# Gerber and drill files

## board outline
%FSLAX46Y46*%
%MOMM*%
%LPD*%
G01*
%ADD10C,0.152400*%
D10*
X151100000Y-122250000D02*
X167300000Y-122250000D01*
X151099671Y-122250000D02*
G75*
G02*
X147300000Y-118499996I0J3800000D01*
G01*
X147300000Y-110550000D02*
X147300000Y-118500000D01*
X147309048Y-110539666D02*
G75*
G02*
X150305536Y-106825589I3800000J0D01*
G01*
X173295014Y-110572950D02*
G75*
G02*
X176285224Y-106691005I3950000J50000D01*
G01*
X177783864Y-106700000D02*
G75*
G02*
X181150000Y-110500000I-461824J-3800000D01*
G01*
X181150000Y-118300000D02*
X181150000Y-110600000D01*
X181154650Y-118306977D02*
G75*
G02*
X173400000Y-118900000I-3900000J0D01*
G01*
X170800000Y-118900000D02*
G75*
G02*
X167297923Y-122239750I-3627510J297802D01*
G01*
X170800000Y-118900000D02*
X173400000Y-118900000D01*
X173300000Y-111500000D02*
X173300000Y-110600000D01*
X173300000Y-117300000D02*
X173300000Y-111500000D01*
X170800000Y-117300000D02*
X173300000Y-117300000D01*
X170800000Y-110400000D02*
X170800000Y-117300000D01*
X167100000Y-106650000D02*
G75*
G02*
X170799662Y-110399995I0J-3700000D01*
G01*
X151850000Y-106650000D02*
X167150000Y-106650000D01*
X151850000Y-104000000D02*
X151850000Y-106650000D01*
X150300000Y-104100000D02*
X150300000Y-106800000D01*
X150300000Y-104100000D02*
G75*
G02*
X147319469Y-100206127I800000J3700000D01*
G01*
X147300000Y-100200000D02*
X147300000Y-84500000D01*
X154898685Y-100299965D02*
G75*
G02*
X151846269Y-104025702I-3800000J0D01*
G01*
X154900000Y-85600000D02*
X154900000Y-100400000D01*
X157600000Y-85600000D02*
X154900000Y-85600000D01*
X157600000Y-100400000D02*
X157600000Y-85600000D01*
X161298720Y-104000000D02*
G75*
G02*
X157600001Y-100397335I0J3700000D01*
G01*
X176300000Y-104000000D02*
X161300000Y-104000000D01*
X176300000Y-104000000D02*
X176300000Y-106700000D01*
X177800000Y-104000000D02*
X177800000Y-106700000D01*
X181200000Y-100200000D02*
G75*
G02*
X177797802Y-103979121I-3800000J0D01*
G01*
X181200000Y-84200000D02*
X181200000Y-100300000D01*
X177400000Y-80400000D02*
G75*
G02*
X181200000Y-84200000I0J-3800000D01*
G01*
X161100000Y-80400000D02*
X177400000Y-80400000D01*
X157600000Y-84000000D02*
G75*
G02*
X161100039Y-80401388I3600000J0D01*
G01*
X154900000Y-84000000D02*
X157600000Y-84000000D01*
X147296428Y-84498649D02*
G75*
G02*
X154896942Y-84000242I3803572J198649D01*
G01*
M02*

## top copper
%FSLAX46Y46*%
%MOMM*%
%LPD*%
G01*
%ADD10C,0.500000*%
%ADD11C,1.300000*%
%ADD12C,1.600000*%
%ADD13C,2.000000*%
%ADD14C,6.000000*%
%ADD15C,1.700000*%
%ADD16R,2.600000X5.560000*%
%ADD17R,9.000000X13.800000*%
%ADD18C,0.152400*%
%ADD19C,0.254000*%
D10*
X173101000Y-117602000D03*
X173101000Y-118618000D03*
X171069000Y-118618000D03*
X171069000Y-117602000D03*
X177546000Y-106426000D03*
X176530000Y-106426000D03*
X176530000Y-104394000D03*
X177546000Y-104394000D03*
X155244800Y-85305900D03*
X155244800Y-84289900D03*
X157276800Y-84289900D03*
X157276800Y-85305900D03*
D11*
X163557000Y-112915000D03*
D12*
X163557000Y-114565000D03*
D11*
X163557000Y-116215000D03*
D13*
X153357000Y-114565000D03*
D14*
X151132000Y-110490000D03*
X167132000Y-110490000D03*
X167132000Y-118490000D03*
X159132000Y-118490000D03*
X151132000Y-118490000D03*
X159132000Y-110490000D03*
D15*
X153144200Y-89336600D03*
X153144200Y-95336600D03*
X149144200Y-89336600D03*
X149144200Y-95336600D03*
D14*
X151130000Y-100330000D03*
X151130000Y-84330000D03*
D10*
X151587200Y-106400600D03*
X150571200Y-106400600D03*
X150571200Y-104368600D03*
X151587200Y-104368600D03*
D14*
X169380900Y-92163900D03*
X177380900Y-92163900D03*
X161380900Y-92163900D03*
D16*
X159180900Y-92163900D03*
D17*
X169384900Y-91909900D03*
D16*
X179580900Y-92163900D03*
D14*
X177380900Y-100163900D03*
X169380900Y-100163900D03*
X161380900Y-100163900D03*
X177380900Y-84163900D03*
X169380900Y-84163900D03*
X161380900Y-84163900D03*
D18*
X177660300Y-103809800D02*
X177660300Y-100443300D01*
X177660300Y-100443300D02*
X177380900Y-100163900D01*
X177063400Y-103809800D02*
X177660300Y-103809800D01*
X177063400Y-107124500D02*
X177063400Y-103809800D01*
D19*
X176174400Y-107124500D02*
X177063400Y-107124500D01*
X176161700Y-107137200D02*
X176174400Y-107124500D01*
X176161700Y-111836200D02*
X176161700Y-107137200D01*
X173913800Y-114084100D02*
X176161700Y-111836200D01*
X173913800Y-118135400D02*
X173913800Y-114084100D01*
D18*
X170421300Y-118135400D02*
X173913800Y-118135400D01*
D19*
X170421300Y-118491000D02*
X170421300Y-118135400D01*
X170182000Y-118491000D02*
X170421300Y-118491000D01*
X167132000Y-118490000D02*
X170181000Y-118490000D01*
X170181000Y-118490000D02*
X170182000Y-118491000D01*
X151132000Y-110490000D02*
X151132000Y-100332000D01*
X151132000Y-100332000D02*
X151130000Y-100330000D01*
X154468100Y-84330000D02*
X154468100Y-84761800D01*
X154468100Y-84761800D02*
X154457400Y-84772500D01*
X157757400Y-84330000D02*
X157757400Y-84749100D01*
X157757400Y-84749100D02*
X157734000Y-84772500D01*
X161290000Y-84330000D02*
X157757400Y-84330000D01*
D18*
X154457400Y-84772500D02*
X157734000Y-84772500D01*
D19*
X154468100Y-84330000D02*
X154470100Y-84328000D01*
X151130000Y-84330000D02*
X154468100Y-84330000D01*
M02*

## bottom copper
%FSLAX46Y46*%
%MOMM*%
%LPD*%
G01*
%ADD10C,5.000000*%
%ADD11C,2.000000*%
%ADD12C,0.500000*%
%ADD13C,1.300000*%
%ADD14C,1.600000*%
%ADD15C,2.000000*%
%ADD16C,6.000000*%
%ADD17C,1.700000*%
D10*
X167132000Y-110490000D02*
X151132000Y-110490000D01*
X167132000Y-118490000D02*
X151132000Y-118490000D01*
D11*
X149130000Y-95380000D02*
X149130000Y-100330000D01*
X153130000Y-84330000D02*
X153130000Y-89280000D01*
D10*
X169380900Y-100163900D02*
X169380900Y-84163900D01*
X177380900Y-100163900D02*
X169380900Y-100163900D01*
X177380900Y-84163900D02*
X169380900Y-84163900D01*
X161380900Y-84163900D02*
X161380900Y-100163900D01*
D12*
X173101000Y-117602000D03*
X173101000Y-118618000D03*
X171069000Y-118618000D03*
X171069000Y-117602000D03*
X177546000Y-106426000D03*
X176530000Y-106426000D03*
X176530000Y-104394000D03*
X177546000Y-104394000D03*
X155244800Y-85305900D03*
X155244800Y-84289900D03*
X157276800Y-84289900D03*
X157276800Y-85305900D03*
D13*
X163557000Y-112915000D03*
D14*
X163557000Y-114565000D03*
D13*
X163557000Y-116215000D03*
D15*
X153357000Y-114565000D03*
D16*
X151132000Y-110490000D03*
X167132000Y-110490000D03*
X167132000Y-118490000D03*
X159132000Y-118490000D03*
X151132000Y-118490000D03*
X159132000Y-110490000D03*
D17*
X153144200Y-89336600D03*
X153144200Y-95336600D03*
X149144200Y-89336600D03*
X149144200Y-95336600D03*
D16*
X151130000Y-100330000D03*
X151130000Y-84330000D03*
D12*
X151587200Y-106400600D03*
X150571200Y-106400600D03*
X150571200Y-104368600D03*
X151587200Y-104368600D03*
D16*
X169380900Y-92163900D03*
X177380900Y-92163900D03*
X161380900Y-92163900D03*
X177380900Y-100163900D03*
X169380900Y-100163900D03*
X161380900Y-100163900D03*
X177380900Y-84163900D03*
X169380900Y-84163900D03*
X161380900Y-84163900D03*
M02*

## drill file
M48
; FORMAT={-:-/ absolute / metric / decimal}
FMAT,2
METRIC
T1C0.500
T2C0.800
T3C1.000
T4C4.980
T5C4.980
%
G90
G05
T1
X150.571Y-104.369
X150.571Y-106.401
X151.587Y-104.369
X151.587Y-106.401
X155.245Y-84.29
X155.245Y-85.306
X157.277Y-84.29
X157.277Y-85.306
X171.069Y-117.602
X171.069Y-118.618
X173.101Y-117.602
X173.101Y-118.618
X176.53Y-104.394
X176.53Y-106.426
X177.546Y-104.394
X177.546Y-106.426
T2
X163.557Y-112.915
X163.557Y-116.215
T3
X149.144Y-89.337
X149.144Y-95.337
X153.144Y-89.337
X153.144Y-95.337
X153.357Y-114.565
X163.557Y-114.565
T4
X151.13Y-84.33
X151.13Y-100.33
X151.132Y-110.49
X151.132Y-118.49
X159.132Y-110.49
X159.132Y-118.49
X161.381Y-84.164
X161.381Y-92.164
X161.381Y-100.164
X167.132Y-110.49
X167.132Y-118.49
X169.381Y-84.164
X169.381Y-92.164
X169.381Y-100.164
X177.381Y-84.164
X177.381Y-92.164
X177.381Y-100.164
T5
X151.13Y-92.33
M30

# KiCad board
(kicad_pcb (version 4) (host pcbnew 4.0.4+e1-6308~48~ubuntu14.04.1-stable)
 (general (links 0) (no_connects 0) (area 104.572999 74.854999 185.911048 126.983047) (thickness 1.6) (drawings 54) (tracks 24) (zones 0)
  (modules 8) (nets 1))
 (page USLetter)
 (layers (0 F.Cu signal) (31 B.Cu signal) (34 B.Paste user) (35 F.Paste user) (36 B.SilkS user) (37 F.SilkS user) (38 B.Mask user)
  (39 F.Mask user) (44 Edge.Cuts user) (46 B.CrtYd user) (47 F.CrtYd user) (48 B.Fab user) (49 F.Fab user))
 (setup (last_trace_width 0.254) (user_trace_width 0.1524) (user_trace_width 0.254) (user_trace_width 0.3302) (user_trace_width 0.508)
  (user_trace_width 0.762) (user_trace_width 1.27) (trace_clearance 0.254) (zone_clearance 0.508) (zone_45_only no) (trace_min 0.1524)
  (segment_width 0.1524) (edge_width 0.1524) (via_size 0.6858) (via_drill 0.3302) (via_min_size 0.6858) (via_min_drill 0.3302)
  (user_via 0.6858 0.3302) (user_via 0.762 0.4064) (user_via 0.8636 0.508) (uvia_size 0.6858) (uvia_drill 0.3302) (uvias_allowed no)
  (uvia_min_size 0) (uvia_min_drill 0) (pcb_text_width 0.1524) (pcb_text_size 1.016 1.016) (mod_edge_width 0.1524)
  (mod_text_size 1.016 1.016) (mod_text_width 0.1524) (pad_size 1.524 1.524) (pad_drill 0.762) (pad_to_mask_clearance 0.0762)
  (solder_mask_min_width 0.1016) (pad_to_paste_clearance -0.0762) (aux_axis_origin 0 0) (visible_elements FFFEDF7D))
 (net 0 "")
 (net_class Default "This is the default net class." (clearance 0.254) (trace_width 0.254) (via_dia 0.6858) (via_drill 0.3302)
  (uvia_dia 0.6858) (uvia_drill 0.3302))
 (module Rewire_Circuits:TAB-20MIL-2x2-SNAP (layer F.Cu) (at 172.085 118.11 270)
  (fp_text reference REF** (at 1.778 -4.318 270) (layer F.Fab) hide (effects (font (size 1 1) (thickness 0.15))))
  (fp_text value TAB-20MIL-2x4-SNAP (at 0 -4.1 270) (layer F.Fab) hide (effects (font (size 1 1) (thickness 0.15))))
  (pad 1 thru_hole circle (at -0.508 -1.016 270) (size 0.5 0.5) (drill 0.5) (layers *.Cu))
  (pad 1 thru_hole circle (at 0.508 -1.016 270) (size 0.5 0.5) (drill 0.5) (layers *.Cu))
  (pad 1 thru_hole circle (at 0.508 1.016 270) (size 0.5 0.5) (drill 0.5) (layers *.Cu))
  (pad 1 thru_hole circle (at -0.508 1.016 270) (size 0.5 0.5) (drill 0.5) (layers *.Cu)))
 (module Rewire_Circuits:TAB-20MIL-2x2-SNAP (layer F.Cu) (at 177.038 105.41 180)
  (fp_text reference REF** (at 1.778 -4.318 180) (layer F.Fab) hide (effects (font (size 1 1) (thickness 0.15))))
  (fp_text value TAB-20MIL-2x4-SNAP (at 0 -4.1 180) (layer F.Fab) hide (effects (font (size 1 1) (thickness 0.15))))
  (pad 1 thru_hole circle (at -0.508 -1.016 180) (size 0.5 0.5) (drill 0.5) (layers *.Cu))
  (pad 1 thru_hole circle (at 0.508 -1.016 180) (size 0.5 0.5) (drill 0.5) (layers *.Cu))
  (pad 1 thru_hole circle (at 0.508 1.016 180) (size 0.5 0.5) (drill 0.5) (layers *.Cu))
  (pad 1 thru_hole circle (at -0.508 1.016 180) (size 0.5 0.5) (drill 0.5) (layers *.Cu)))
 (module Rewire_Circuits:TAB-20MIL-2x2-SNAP (layer F.Cu) (at 156.2608 84.7979 90)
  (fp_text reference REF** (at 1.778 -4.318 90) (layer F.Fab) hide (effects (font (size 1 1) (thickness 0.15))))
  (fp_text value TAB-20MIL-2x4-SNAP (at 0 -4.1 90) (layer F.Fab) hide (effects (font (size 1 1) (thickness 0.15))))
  (pad 1 thru_hole circle (at -0.508 -1.016 90) (size 0.5 0.5) (drill 0.5) (layers *.Cu))
  (pad 1 thru_hole circle (at 0.508 -1.016 90) (size 0.5 0.5) (drill 0.5) (layers *.Cu))
  (pad 1 thru_hole circle (at 0.508 1.016 90) (size 0.5 0.5) (drill 0.5) (layers *.Cu))
  (pad 1 thru_hole circle (at -0.508 1.016 90) (size 0.5 0.5) (drill 0.5) (layers *.Cu)))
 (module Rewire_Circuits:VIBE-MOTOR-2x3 (layer F.Cu) (at 167.132 110.49 180)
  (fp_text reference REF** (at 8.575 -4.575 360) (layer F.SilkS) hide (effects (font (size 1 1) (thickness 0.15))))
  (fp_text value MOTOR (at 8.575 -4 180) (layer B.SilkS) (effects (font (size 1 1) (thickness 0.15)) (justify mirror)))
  (fp_line (start 0 0) (end 16 0) (layer B.Cu) (width 5)) (fp_line (start 0 -8) (end 16 -8) (layer B.Cu) (width 5))
  (pad 1 thru_hole circle (at 3.575 -2.425 270) (size 1.3 1.3) (drill 0.8) (layers *.Cu *.Mask F.SilkS))
  (pad 3 thru_hole circle (at 3.575 -4.075 270) (size 1.6 1.6) (drill 1) (layers *.Cu *.Mask F.SilkS))
  (pad 2 thru_hole circle (at 3.575 -5.725 270) (size 1.3 1.3) (drill 0.8) (layers *.Cu *.Mask F.SilkS))
  (pad 3 thru_hole circle (at 13.775 -4.075 270) (size 2 2) (drill 1) (layers *.Cu *.Mask F.SilkS))
  (pad 1 thru_hole circle (at 16 0 180) (size 6 6) (drill 4.98) (layers *.Cu *.Mask))
  (pad 1 thru_hole circle (at 0 0 180) (size 6 6) (drill 4.98) (layers *.Cu *.Mask))
  (pad 2 thru_hole circle (at 0 -8 180) (size 6 6) (drill 4.98) (layers *.Cu *.Mask))
  (pad 2 thru_hole circle (at 8 -8 180) (size 6 6) (drill 4.98) (layers *.Cu *.Mask))
  (pad 2 thru_hole circle (at 16 -8 180) (size 6 6) (drill 4.98) (layers *.Cu *.Mask))
  (pad 1 thru_hole circle (at 8 0 180) (size 6 6) (drill 4.98) (layers *.Cu *.Mask)))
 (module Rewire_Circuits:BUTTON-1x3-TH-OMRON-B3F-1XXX (layer F.Cu) (at 151.13 100.33 90)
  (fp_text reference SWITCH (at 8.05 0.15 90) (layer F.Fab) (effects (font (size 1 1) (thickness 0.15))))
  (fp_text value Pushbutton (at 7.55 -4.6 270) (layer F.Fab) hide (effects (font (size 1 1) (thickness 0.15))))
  (fp_line (start 4.95 -2) (end 0 -2) (layer B.Cu) (width 2)) (fp_line (start 16 2) (end 11.05 2) (layer B.Cu) (width 2))
  (pad 2 thru_hole circle (at 10.9934 2.0142 90) (size 1.7 1.7) (drill 1) (layers *.Cu *.Mask))
  (pad 2 thru_hole circle (at 4.9934 2.0142 90) (size 1.7 1.7) (drill 1) (layers *.Cu *.Mask))
  (pad 1 thru_hole circle (at 10.9934 -1.9858 90) (size 1.7 1.7) (drill 1) (layers *.Cu *.Mask))
  (pad 1 thru_hole circle (at 4.9934 -1.9858 90) (size 1.7 1.7) (drill 1) (layers *.Cu *.Mask))
  (pad "" np_thru_hole circle (at 8 0 90) (size 4.88 4.88) (drill 4.98) (layers *.Cu *.Mask F.SilkS))
  (pad 1 thru_hole circle (at 0 0 90) (size 6 6) (drill 4.98) (layers *.Cu *.Mask F.SilkS))
  (pad 2 thru_hole circle (at 16 0 90) (size 6 6) (drill 4.98) (layers *.Cu *.Mask F.SilkS)))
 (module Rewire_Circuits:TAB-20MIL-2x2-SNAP (layer F.Cu) (at 151.0792 105.3846 180)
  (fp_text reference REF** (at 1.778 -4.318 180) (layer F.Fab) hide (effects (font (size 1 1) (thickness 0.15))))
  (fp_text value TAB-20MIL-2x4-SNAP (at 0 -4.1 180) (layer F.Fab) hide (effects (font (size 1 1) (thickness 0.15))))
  (pad 1 thru_hole circle (at -0.508 -1.016 180) (size 0.5 0.5) (drill 0.5) (layers *.Cu))
  (pad 1 thru_hole circle (at 0.508 -1.016 180) (size 0.5 0.5) (drill 0.5) (layers *.Cu))
  (pad 1 thru_hole circle (at 0.508 1.016 180) (size 0.5 0.5) (drill 0.5) (layers *.Cu))
  (pad 1 thru_hole circle (at -0.508 1.016 180) (size 0.5 0.5) (drill 0.5) (layers *.Cu)))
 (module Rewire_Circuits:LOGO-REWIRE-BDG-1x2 (layer F.Cu) (at 181.1528 114.427 90)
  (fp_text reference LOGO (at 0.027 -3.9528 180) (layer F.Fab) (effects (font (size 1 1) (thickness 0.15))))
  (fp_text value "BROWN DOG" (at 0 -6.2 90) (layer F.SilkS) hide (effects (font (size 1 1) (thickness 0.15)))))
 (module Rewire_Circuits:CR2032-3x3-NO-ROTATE (layer F.Cu) (at 177.3809 84.1639 180)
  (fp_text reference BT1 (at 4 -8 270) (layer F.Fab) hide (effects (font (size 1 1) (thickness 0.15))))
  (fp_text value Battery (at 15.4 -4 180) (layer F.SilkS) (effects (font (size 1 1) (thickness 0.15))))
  (fp_line (start 8 -16) (end 8 0) (layer B.Cu) (width 5)) (fp_line (start 0 -16) (end 8 -16) (layer B.Cu) (width 5))
  (fp_line (start 0 0) (end 8 0) (layer B.Cu) (width 5)) (fp_line (start 16 0) (end 16 -16) (layer B.Cu) (width 5))
  (pad GND thru_hole circle (at 8 -8 180) (size 6 6) (drill 4.98) (layers *.Cu *.Mask))
  (pad + thru_hole circle (at 0 -8 180) (size 6 6) (drill 4.98) (layers *.Cu *.Mask))
  (pad + thru_hole circle (at 16 -8 180) (size 6 6) (drill 4.98) (layers *.Cu *.Mask))
  (pad + smd rect (at 18.2 -8 180) (size 2.6 5.56) (layers F.Cu F.Paste F.Mask))
  (pad GND smd rect (at 7.996 -7.746 180) (size 9 13.8) (layers F.Cu F.Paste F.Mask))
  (pad + smd rect (at -2.2 -8 180) (size 2.6 5.56) (layers F.Cu F.Paste F.Mask))
  (pad GND thru_hole circle (at 0 -16 180) (size 6 6) (drill 4.98) (layers *.Cu *.Mask))
  (pad GND thru_hole circle (at 8 -16 180) (size 6 6) (drill 4.98) (layers *.Cu *.Mask))
  (pad + thru_hole circle (at 16 -16 180) (size 6 6) (drill 4.98) (layers *.Cu B.Mask))
  (pad GND thru_hole circle (at 0 0 180) (size 6 6) (drill 4.98) (layers *.Cu *.Mask))
  (pad GND thru_hole circle (at 8 0 180) (size 6 6) (drill 4.98) (layers *.Cu *.Mask))
  (pad + thru_hole circle (at 16 0 180) (size 6 6) (drill 4.98) (layers *.Cu B.Mask)))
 (gr_line (start 151.1 122.25) (end 167.3 122.25) (layer Edge.Cuts) (width 0.1524))
 (gr_arc (start 151.099671 118.45) (end 151.099671 122.25) (angle 89.24615167) (layer Edge.Cuts) (width 0.1524))
 (gr_line (start 147.3 110.55) (end 147.3 118.5) (layer Edge.Cuts) (width 0.1524))
 (gr_arc (start 151.109048 110.539666) (end 147.309048 110.539666) (angle 77.79262944) (layer Edge.Cuts) (width 0.1524))
 (gr_arc (start 177.245014 110.52295) (end 173.295014 110.57295) (angle 76.66359666) (layer Edge.Cuts) (width 0.1524))
 (gr_arc (start 177.32204 110.5) (end 177.783864 106.7) (angle 83.07067559) (layer Edge.Cuts) (width 0.1524))
 (gr_line (start 181.15 118.3) (end 181.15 110.6) (layer Edge.Cuts) (width 0.1524))
 (gr_arc (start 177.25465 118.306977) (end 181.15465 118.306977) (angle 171.2538377) (layer Edge.Cuts) (width 0.1524))
 (gr_arc (start 167.17249 118.602198) (end 170.8 118.9) (angle 83.33186569) (layer Edge.Cuts) (width 0.1524))
 (gr_line (start 170.8 118.9) (end 173.4 118.9) (layer Edge.Cuts) (width 0.1524))
 (gr_line (start 173.3 111.5) (end 173.3 110.6) (layer Edge.Cuts) (width 0.1524))
 (gr_line (start 173.3 117.3) (end 173.3 111.5) (layer Edge.Cuts) (width 0.1524))
 (gr_line (start 170.8 117.3) (end 173.3 117.3) (layer Edge.Cuts) (width 0.1524))
 (gr_line (start 170.8 110.4) (end 170.8 117.3) (layer Edge.Cuts) (width 0.1524))
 (gr_arc (start 167.1 110.35) (end 167.1 106.65) (angle 90.77421347) (layer Edge.Cuts) (width 0.1524))
 (gr_line (start 151.85 106.65) (end 167.15 106.65) (layer Edge.Cuts) (width 0.1524))
 (gr_line (start 151.85 104) (end 151.85 106.65) (layer Edge.Cuts) (width 0.1524))
 (gr_line (start 150.3 104.1) (end 150.3 106.8) (layer Edge.Cuts) (width 0.1524))
 (gr_arc (start 151.1 100.4) (end 150.3 104.1) (angle 80.73520472) (layer Edge.Cuts) (width 0.1524))
 (gr_line (start 147.3 100.2) (end 147.3 84.5) (layer Edge.Cuts) (width 0.1524))
 (gr_arc (start 151.098685 100.299965) (end 154.898685 100.299965) (angle 78.6540423) (layer Edge.Cuts) (width 0.1524))
 (gr_line (start 154.9 85.6) (end 154.9 100.4) (layer Edge.Cuts) (width 0.1524))
 (gr_line (start 157.6 85.6) (end 154.9 85.6) (layer Edge.Cuts) (width 0.1524))
 (gr_line (start 157.6 100.4) (end 157.6 85.6) (layer Edge.Cuts) (width 0.1524))
 (gr_arc (start 161.29872 100.3) (end 161.29872 104) (angle 88.49256424) (layer Edge.Cuts) (width 0.1524))
 (gr_line (start 176.3 104) (end 161.3 104) (layer Edge.Cuts) (width 0.1524))
 (gr_line (start 176.3 104) (end 176.3 106.7) (layer Edge.Cuts) (width 0.1524))
 (gr_line (start 177.8 104) (end 177.8 106.7) (layer Edge.Cuts) (width 0.1524))
 (gr_arc (start 177.4 100.2) (end 181.2 100.2) (angle 83.99099562) (layer Edge.Cuts) (width 0.1524))
 (gr_line (start 181.2 84.2) (end 181.2 100.3) (layer Edge.Cuts) (width 0.1524))
 (gr_arc (start 177.4 84.2) (end 177.4 80.4) (angle 90) (layer Edge.Cuts) (width 0.1524))
 (gr_line (start 161.1 80.4) (end 177.4 80.4) (layer Edge.Cuts) (width 0.1524))
 (gr_arc (start 161.2 84) (end 157.6 84) (angle 88.40885973) (layer Edge.Cuts) (width 0.1524))
 (gr_line (start 154.9 84) (end 157.6 84) (layer Edge.Cuts) (width 0.1524))
 (gr_arc (start 151.1 84.3) (end 147.296428 84.498649) (angle 178.4756859) (layer Edge.Cuts) (width 0.1524))
 (segment (start 177.6603 103.8098) (end 177.6603 100.4433) (width 0.1524) (layer F.Cu) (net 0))
 (segment (start 177.6603 100.4433) (end 177.3809 100.1639) (width 0.1524) (layer F.Cu) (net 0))
 (segment (start 177.0634 103.8098) (end 177.6603 103.8098) (width 0.1524) (layer F.Cu) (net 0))
 (segment (start 177.0634 107.1245) (end 177.0634 103.8098) (width 0.1524) (layer F.Cu) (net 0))
 (segment (start 176.1744 107.1245) (end 177.0634 107.1245) (width 0.254) (layer F.Cu) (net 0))
 (segment (start 176.1617 107.1372) (end 176.1744 107.1245) (width 0.254) (layer F.Cu) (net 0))
 (segment (start 176.1617 111.8362) (end 176.1617 107.1372) (width 0.254) (layer F.Cu) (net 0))
 (segment (start 173.9138 114.0841) (end 176.1617 111.8362) (width 0.254) (layer F.Cu) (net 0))
 (segment (start 173.9138 118.1354) (end 173.9138 114.0841) (width 0.254) (layer F.Cu) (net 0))
 (segment (start 170.4213 118.1354) (end 173.9138 118.1354) (width 0.1524) (layer F.Cu) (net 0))
 (segment (start 170.4213 118.491) (end 170.4213 118.1354) (width 0.254) (layer F.Cu) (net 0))
 (segment (start 170.182 118.491) (end 170.4213 118.491) (width 0.254) (layer F.Cu) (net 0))
 (segment (start 167.132 118.49) (end 170.181 118.49) (width 0.254) (layer F.Cu) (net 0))
 (segment (start 170.181 118.49) (end 170.182 118.491) (width 0.254) (layer F.Cu) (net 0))
 (segment (start 151.132 110.49) (end 151.132 100.332) (width 0.254) (layer F.Cu) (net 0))
 (segment (start 151.132 100.332) (end 151.13 100.33) (width 0.254) (layer F.Cu) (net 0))
 (segment (start 154.4681 84.33) (end 154.4681 84.7618) (width 0.254) (layer F.Cu) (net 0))
 (segment (start 154.4681 84.7618) (end 154.4574 84.7725) (width 0.254) (layer F.Cu) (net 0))
 (segment (start 157.7574 84.33) (end 157.7574 84.7491) (width 0.254) (layer F.Cu) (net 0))
 (segment (start 157.7574 84.7491) (end 157.734 84.7725) (width 0.254) (layer F.Cu) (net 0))
 (segment (start 161.29 84.33) (end 157.7574 84.33) (width 0.254) (layer F.Cu) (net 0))
 (segment (start 154.4574 84.7725) (end 157.734 84.7725) (width 0.1524) (layer F.Cu) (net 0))
 (segment (start 154.4681 84.33) (end 154.4701 84.328) (width 0.254) (layer F.Cu) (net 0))
 (segment (start 151.13 84.33) (end 154.4681 84.33) (width 0.254) (layer F.Cu) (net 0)))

